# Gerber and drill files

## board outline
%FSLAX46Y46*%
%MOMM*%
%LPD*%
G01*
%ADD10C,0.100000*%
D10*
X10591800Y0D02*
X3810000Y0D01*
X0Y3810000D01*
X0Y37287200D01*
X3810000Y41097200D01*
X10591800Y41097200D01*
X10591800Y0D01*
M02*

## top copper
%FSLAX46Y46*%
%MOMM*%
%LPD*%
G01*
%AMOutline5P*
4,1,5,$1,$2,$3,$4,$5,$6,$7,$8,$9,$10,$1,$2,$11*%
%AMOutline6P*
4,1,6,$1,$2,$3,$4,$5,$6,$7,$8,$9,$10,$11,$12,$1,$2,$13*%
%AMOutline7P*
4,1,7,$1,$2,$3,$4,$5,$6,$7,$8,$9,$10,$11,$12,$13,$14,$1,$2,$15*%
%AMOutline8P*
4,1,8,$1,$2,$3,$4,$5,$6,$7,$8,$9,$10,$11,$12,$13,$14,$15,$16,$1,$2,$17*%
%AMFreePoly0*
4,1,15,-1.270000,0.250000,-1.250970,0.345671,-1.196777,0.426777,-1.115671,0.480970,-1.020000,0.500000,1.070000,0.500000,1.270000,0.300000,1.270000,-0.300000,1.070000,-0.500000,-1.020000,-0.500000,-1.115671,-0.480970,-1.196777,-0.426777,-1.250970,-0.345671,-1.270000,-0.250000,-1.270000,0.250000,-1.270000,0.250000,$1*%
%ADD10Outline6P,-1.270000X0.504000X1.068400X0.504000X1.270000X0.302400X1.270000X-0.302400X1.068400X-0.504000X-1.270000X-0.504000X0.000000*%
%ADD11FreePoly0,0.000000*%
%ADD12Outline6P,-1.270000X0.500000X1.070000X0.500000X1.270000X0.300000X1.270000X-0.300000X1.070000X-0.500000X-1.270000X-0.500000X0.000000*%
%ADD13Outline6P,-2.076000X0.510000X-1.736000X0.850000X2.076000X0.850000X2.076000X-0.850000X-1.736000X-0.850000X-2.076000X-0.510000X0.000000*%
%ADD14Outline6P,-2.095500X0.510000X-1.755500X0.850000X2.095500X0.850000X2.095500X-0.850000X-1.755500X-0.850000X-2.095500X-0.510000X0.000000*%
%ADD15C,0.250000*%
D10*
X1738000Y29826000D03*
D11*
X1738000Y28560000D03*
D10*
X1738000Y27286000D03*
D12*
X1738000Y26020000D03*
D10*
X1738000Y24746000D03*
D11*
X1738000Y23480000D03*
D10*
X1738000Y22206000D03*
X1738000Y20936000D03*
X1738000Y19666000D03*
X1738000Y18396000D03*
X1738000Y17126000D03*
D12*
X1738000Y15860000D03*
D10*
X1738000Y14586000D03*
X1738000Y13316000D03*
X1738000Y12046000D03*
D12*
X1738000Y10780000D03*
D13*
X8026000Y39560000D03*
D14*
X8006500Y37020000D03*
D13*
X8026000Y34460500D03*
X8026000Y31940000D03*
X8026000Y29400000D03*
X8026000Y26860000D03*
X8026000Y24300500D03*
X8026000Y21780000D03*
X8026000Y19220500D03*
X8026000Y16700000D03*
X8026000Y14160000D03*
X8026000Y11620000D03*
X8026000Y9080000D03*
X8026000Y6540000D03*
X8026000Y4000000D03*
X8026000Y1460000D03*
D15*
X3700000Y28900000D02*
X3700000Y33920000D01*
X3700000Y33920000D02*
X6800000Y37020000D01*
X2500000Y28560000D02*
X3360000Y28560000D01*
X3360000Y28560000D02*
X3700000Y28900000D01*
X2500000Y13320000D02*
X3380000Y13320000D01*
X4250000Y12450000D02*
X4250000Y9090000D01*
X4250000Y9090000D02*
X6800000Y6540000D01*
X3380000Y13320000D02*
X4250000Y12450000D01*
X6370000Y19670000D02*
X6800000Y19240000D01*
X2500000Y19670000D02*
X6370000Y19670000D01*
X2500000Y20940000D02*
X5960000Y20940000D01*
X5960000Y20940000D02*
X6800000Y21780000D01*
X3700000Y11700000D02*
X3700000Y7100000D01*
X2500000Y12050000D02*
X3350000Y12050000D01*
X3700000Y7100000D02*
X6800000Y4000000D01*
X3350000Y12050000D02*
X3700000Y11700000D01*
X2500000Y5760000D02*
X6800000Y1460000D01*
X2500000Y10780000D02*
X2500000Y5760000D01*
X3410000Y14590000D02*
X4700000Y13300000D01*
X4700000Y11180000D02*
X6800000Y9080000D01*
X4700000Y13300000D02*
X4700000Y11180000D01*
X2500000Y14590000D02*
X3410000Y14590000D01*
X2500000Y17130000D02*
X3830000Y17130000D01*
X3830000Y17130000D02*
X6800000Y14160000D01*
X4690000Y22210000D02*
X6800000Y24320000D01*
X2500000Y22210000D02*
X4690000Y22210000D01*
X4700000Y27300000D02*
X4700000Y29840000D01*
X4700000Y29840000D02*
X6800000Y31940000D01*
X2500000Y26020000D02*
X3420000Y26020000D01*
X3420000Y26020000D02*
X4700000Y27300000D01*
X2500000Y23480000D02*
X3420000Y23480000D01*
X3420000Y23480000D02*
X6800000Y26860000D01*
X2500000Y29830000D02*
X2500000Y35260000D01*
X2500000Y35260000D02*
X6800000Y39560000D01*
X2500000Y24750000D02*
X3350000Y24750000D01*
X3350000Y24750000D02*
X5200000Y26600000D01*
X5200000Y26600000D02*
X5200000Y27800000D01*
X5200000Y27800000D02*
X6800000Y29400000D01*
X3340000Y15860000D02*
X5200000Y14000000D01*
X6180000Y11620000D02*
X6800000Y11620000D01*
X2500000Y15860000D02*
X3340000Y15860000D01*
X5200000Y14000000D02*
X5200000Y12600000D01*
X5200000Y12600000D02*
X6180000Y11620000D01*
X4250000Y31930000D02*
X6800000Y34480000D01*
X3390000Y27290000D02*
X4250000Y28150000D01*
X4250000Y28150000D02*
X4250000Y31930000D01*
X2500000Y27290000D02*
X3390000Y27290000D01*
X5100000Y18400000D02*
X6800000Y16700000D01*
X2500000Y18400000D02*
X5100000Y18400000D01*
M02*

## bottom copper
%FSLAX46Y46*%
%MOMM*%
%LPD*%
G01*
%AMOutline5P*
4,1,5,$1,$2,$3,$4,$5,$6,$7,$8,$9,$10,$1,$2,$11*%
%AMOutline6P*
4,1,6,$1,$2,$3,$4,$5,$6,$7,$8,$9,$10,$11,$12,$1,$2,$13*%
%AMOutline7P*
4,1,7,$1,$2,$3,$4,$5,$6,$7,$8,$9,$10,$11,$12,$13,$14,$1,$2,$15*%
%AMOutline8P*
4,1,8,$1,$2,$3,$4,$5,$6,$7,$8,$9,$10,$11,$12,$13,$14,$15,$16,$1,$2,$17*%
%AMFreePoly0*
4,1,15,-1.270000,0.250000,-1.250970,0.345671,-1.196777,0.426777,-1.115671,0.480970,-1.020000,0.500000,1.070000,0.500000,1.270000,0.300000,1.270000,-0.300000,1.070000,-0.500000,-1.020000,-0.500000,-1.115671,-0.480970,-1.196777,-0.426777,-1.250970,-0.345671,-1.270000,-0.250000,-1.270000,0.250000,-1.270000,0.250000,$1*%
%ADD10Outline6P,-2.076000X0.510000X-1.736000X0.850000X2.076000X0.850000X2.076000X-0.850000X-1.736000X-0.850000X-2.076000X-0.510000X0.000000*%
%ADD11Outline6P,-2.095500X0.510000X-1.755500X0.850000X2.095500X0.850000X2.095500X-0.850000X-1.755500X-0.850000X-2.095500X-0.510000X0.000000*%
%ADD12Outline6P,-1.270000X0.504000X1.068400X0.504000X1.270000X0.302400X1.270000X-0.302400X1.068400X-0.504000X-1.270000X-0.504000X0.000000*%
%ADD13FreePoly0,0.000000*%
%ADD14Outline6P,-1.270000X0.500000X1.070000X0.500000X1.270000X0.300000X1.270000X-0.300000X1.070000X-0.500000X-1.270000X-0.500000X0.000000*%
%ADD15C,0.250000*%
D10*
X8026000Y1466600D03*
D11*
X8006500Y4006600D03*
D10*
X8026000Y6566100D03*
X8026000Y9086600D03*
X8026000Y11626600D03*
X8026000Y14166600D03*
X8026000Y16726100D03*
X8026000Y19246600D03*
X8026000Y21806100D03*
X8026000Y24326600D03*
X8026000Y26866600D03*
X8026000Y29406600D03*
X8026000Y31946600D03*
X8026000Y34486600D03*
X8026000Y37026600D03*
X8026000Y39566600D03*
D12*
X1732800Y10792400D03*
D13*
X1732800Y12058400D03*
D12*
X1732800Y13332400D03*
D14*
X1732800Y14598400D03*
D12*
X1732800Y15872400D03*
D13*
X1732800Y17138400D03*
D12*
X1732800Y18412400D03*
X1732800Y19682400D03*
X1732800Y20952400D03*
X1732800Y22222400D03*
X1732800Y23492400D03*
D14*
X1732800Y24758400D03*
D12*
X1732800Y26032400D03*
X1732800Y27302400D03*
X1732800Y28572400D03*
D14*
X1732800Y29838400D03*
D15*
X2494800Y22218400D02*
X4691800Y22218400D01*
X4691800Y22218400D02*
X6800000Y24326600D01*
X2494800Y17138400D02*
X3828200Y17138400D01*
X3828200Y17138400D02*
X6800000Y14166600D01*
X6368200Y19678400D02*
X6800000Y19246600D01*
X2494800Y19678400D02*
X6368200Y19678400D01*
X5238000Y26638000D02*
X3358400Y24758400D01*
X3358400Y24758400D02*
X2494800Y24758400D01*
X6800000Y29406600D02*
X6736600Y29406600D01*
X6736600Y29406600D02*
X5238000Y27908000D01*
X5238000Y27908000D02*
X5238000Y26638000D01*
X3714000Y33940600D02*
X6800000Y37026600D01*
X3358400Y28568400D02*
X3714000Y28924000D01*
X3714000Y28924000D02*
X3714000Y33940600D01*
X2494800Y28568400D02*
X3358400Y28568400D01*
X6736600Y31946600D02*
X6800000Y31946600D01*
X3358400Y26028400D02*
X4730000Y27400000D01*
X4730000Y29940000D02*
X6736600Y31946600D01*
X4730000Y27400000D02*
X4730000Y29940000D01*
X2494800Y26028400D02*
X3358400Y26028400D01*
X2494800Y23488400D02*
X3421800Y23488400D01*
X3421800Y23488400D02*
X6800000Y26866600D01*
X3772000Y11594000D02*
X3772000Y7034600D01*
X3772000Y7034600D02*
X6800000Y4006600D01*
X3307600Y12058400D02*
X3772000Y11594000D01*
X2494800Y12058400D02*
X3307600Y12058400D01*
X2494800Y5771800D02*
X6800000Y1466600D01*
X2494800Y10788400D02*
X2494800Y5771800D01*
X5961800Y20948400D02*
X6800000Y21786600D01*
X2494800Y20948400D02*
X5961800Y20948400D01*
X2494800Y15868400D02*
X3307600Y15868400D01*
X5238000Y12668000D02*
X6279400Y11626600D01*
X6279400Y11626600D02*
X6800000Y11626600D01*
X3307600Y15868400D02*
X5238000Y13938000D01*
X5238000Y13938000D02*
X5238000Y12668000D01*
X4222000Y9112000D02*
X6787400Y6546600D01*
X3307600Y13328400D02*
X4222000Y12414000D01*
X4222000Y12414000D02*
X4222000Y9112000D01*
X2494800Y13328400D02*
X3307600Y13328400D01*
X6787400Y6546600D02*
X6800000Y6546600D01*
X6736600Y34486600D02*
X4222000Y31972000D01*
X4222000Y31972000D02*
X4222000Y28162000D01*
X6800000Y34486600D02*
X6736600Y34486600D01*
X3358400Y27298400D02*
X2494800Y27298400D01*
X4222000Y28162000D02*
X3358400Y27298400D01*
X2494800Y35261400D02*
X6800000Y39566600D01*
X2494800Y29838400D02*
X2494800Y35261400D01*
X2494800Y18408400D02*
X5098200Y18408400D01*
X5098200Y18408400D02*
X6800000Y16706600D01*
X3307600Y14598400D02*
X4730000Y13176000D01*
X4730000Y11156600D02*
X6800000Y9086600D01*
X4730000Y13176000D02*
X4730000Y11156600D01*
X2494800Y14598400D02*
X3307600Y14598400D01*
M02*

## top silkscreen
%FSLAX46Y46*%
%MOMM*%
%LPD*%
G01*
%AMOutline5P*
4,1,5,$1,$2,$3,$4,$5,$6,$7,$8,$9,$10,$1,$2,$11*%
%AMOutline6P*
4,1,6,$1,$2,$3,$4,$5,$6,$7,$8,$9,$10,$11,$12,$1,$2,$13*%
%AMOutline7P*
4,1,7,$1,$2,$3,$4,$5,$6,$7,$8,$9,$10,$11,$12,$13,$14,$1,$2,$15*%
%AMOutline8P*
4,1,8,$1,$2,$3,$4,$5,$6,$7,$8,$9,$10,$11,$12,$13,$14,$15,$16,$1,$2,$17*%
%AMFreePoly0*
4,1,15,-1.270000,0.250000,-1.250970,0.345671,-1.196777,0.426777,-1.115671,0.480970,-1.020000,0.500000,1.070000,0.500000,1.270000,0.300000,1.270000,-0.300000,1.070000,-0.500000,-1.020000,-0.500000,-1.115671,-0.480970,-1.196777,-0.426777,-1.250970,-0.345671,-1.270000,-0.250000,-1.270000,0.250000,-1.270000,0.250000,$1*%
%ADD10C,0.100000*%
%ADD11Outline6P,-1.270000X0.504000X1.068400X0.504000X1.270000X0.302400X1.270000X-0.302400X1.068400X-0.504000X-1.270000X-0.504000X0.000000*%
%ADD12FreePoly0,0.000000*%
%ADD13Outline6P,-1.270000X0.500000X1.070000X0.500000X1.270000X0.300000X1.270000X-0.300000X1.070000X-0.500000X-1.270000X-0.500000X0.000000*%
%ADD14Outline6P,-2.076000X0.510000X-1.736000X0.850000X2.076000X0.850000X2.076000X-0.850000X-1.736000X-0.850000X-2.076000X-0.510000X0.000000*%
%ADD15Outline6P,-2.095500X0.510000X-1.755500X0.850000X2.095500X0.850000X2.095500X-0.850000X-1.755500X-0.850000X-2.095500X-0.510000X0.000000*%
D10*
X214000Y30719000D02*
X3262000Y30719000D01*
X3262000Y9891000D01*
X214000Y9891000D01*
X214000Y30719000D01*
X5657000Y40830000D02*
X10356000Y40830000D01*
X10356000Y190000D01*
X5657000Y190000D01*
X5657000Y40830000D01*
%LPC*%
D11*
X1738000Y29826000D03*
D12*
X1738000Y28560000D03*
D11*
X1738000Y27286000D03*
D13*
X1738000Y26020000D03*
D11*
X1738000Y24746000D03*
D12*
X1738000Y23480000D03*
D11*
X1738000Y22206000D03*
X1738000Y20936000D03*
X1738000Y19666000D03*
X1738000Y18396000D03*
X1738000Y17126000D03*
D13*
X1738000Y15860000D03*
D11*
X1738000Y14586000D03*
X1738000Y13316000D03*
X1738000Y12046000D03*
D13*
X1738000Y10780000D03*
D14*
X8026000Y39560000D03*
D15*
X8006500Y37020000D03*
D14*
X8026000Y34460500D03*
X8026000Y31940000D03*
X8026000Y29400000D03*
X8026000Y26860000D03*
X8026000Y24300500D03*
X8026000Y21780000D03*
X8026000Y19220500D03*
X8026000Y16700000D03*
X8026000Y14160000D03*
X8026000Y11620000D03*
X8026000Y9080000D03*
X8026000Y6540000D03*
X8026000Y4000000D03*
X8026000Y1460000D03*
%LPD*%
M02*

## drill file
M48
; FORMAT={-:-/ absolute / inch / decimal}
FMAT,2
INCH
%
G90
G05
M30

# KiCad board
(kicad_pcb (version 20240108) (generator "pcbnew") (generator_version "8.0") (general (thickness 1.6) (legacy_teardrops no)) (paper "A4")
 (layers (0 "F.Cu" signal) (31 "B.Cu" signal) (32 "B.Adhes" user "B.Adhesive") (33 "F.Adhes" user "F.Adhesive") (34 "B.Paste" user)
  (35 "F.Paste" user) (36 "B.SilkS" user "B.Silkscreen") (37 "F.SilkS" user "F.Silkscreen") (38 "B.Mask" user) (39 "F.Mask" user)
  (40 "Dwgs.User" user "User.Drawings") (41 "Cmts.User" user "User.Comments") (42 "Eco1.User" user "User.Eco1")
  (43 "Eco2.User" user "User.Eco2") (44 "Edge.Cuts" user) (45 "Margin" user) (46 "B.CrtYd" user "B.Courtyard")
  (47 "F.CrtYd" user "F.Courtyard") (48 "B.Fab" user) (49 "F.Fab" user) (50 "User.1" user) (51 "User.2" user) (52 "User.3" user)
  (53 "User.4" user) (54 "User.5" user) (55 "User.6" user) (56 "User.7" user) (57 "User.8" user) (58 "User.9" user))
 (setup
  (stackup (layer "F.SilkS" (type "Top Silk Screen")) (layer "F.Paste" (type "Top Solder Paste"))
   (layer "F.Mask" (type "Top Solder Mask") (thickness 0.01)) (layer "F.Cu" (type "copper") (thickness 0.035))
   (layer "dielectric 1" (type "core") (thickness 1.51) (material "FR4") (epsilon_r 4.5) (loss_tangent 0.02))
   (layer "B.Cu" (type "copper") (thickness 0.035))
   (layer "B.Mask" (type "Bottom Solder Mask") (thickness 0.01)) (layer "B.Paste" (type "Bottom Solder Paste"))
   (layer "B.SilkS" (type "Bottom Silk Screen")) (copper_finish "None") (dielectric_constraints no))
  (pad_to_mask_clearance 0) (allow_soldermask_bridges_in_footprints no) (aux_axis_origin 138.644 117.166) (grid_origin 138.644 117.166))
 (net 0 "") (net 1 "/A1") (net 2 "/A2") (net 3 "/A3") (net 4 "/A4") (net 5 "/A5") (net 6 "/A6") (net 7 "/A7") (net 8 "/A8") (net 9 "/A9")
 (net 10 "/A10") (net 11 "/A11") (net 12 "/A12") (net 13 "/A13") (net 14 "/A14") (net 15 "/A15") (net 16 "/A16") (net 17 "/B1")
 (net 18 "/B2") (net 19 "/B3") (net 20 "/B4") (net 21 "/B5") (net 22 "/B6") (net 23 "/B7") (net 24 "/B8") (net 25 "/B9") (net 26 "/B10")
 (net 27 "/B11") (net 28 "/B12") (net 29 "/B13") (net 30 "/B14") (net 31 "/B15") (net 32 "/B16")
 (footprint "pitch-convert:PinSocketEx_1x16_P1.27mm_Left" (layer "F.Cu") (at 139.62 87.336)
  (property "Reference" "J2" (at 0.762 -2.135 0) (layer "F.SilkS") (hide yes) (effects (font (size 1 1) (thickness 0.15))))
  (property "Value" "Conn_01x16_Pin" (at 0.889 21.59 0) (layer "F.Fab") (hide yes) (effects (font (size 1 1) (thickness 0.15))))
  (fp_rect (start -0.762 -0.889) (end 2.286 19.939) (stroke (width 0.1) (type default)) (fill none) (layer "F.SilkS"))
  (pad "1" smd roundrect (at 1.524 0) (size 2.54 1.008) (drill (offset -0.762 0.004)) (layers "F.Cu" "F.Paste" "F.Mask")
   (roundrect_rratio 0) (chamfer_ratio 0.2) (chamfer top_right bottom_right) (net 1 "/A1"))
  (pad "2" smd roundrect (at 1.524 1.27) (size 2.54 1) (drill (offset -0.762 0)) (layers "F.Cu" "F.Paste" "F.Mask") (roundrect_rratio 0.25)
   (chamfer_ratio 0.2) (chamfer top_right bottom_right) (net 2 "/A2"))
  (pad "3" smd roundrect (at 1.524 2.54) (size 2.54 1.008) (drill (offset -0.762 0.004)) (layers "F.Cu" "F.Paste" "F.Mask")
   (roundrect_rratio 0) (chamfer_ratio 0.2) (chamfer top_right bottom_right) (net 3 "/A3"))
  (pad "4" smd roundrect (at 1.524 3.81) (size 2.54 1) (drill (offset -0.762 0)) (layers "F.Cu" "F.Paste" "F.Mask") (roundrect_rratio 0)
   (chamfer_ratio 0.2) (chamfer top_right bottom_right) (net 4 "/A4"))
  (pad "5" smd roundrect (at 1.524 5.08) (size 2.54 1.008) (drill (offset -0.762 0.004)) (layers "F.Cu" "F.Paste" "F.Mask")
   (roundrect_rratio 0) (chamfer_ratio 0.2) (chamfer top_right bottom_right) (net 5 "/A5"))
  (pad "6" smd roundrect (at 1.524 6.35) (size 2.54 1) (drill (offset -0.762 0)) (layers "F.Cu" "F.Paste" "F.Mask") (roundrect_rratio 0.25)
   (chamfer_ratio 0.2) (chamfer top_right bottom_right) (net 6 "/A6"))
  (pad "7" smd roundrect (at 1.524 7.62) (size 2.54 1.008) (drill (offset -0.762 0.004)) (layers "F.Cu" "F.Paste" "F.Mask")
   (roundrect_rratio 0) (chamfer_ratio 0.2) (chamfer top_right bottom_right) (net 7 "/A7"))
  (pad "8" smd roundrect (at 1.524 8.89) (size 2.54 1.008) (drill (offset -0.762 0.004)) (layers "F.Cu" "F.Paste" "F.Mask")
   (roundrect_rratio 0) (chamfer_ratio 0.2) (chamfer top_right bottom_right) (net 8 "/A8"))
  (pad "9" smd roundrect (at 1.524 10.16) (size 2.54 1.008) (drill (offset -0.762 0.004)) (layers "F.Cu" "F.Paste" "F.Mask")
   (roundrect_rratio 0) (chamfer_ratio 0.2) (chamfer top_right bottom_right) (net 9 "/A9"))
  (pad "10" smd roundrect (at 1.524 11.43) (size 2.54 1.008) (drill (offset -0.762 0.004)) (layers "F.Cu" "F.Paste" "F.Mask")
   (roundrect_rratio 0) (chamfer_ratio 0.2) (chamfer top_right bottom_right) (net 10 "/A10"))
  (pad "11" smd roundrect (at 1.524 12.7) (size 2.54 1.008) (drill (offset -0.762 0.004)) (layers "F.Cu" "F.Paste" "F.Mask")
   (roundrect_rratio 0) (chamfer_ratio 0.2) (chamfer top_right bottom_right) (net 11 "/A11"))
  (pad "12" smd roundrect (at 1.524 13.97) (size 2.54 1) (drill (offset -0.762 0)) (layers "F.Cu" "F.Paste" "F.Mask") (roundrect_rratio 0)
   (chamfer_ratio 0.2) (chamfer top_right bottom_right) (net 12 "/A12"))
  (pad "13" smd roundrect (at 1.524 15.24) (size 2.54 1.008) (drill (offset -0.762 0.004)) (layers "F.Cu" "F.Paste" "F.Mask")
   (roundrect_rratio 0) (chamfer_ratio 0.2) (chamfer top_right bottom_right) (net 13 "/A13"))
  (pad "14" smd roundrect (at 1.524 16.51) (size 2.54 1.008) (drill (offset -0.762 0.004)) (layers "F.Cu" "F.Paste" "F.Mask")
   (roundrect_rratio 0) (chamfer_ratio 0.2) (chamfer top_right bottom_right) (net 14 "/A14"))
  (pad "15" smd roundrect (at 1.524 17.78) (size 2.54 1.008) (drill (offset -0.762 0.004)) (layers "F.Cu" "F.Paste" "F.Mask")
   (roundrect_rratio 0) (chamfer_ratio 0.2) (chamfer top_right bottom_right) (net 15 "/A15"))
  (pad "16" smd roundrect (at 1.524 19.05) (size 2.54 1) (drill (offset -0.762 0)) (layers "F.Cu" "F.Paste" "F.Mask") (roundrect_rratio 0)
   (chamfer_ratio 0.2) (chamfer top_right bottom_right) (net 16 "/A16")))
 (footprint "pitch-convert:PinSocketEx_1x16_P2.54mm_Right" (layer "F.Cu") (at 145.444 77.606)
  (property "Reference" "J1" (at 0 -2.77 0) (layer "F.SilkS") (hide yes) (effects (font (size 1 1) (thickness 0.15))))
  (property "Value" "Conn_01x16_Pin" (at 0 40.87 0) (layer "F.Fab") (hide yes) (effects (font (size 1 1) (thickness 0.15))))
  (fp_rect (start -1.143 -1.27) (end 3.556 39.37) (stroke (width 0.1) (type default)) (fill none) (layer "F.SilkS"))
  (pad "1" smd roundrect (at 0 0) (size 4.152 1.7) (drill (offset 1.226 0)) (layers "F.Cu" "F.Paste" "F.Mask") (roundrect_rratio 0)
   (chamfer_ratio 0.2) (chamfer top_left bottom_left) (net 1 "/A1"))
  (pad "2" smd roundrect (at 0 2.54) (size 4.191 1.7) (drill (offset 1.2065 0)) (layers "F.Cu" "F.Paste" "F.Mask") (roundrect_rratio 0)
   (chamfer_ratio 0.2) (chamfer top_left bottom_left) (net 2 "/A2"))
  (pad "3" smd roundrect (at 0 5.08) (size 4.152 1.7) (drill (offset 1.226 0.0195)) (layers "F.Cu" "F.Paste" "F.Mask") (roundrect_rratio 0)
   (chamfer_ratio 0.2) (chamfer top_left bottom_left) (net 3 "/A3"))
  (pad "4" smd roundrect (at 0 7.62) (size 4.152 1.7) (drill (offset 1.226 0)) (layers "F.Cu" "F.Paste" "F.Mask") (roundrect_rratio 0)
   (chamfer_ratio 0.2) (chamfer top_left bottom_left) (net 4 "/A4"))
  (pad "5" smd roundrect (at 0 10.16) (size 4.152 1.7) (drill (offset 1.226 0)) (layers "F.Cu" "F.Paste" "F.Mask") (roundrect_rratio 0)
   (chamfer_ratio 0.2) (chamfer top_left bottom_left) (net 5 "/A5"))
  (pad "6" smd roundrect (at 0 12.7) (size 4.152 1.7) (drill (offset 1.226 0)) (layers "F.Cu" "F.Paste" "F.Mask") (roundrect_rratio 0)
   (chamfer_ratio 0.2) (chamfer top_left bottom_left) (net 6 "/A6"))
  (pad "7" smd roundrect (at 0 15.24) (size 4.152 1.7) (drill (offset 1.226 0.0195)) (layers "F.Cu" "F.Paste" "F.Mask") (roundrect_rratio 0)
   (chamfer_ratio 0.2) (chamfer top_left bottom_left) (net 7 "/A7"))
  (pad "8" smd roundrect (at 0 17.78) (size 4.152 1.7) (drill (offset 1.226 0)) (layers "F.Cu" "F.Paste" "F.Mask") (roundrect_rratio 0)
   (chamfer_ratio 0.2) (chamfer top_left bottom_left) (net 8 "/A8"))
  (pad "9" smd roundrect (at 0 20.32) (size 4.152 1.7) (drill (offset 1.226 0.0195)) (layers "F.Cu" "F.Paste" "F.Mask") (roundrect_rratio 0)
   (chamfer_ratio 0.2) (chamfer top_left bottom_left) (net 9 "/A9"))
  (pad "10" smd roundrect (at 0 22.86) (size 4.152 1.7) (drill (offset 1.226 0)) (layers "F.Cu" "F.Paste" "F.Mask") (roundrect_rratio 0)
   (chamfer_ratio 0.2) (chamfer top_left bottom_left) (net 10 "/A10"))
  (pad "11" smd roundrect (at 0 25.4) (size 4.152 1.7) (drill (offset 1.226 0)) (layers "F.Cu" "F.Paste" "F.Mask") (roundrect_rratio 0)
   (chamfer_ratio 0.2) (chamfer top_left bottom_left) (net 11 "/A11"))
  (pad "12" smd roundrect (at 0 27.94) (size 4.152 1.7) (drill (offset 1.226 0)) (layers "F.Cu" "F.Paste" "F.Mask") (roundrect_rratio 0)
   (chamfer_ratio 0.2) (chamfer top_left bottom_left) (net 12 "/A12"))
  (pad "13" smd roundrect (at 0 30.48) (size 4.152 1.7) (drill (offset 1.226 0)) (layers "F.Cu" "F.Paste" "F.Mask") (roundrect_rratio 0)
   (chamfer_ratio 0.2) (chamfer top_left bottom_left) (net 13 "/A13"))
  (pad "14" smd roundrect (at 0 33.02) (size 4.152 1.7) (drill (offset 1.226 0)) (layers "F.Cu" "F.Paste" "F.Mask") (roundrect_rratio 0)
   (chamfer_ratio 0.2) (chamfer top_left bottom_left) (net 14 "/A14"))
  (pad "15" smd roundrect (at 0 35.56) (size 4.152 1.7) (drill (offset 1.226 0)) (layers "F.Cu" "F.Paste" "F.Mask") (roundrect_rratio 0)
   (chamfer_ratio 0.2) (chamfer top_left bottom_left) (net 15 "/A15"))
  (pad "16" smd roundrect (at 0 38.1) (size 4.152 1.7) (drill (offset 1.226 0)) (layers "F.Cu" "F.Paste" "F.Mask") (roundrect_rratio 0)
   (chamfer_ratio 0.2) (chamfer top_left bottom_left) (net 16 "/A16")))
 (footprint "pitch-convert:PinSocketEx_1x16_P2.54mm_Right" (layer "B.Cu") (at 145.444 115.6994)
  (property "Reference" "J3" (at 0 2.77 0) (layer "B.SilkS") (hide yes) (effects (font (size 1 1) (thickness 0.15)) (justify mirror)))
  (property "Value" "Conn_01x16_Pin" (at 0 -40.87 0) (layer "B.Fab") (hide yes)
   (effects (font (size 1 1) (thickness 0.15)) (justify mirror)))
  (pad "1" smd roundrect (at 0 0) (size 4.152 1.7) (drill (offset 1.226 0)) (layers "B.Cu" "B.Paste" "B.Mask") (roundrect_rratio 0)
   (chamfer_ratio 0.2) (chamfer top_left bottom_left) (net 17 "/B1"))
  (pad "2" smd roundrect (at 0 -2.54) (size 4.191 1.7) (drill (offset 1.2065 0)) (layers "B.Cu" "B.Paste" "B.Mask") (roundrect_rratio 0)
   (chamfer_ratio 0.2) (chamfer top_left bottom_left) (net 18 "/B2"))
  (pad "3" smd roundrect (at 0 -5.08) (size 4.152 1.7) (drill (offset 1.226 -0.0195)) (layers "B.Cu" "B.Paste" "B.Mask")
   (roundrect_rratio 0) (chamfer_ratio 0.2) (chamfer top_left bottom_left) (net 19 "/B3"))
  (pad "4" smd roundrect (at 0 -7.62) (size 4.152 1.7) (drill (offset 1.226 0)) (layers "B.Cu" "B.Paste" "B.Mask") (roundrect_rratio 0)
   (chamfer_ratio 0.2) (chamfer top_left bottom_left) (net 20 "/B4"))
  (pad "5" smd roundrect (at 0 -10.16) (size 4.152 1.7) (drill (offset 1.226 0)) (layers "B.Cu" "B.Paste" "B.Mask") (roundrect_rratio 0)
   (chamfer_ratio 0.2) (chamfer top_left bottom_left) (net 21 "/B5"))
  (pad "6" smd roundrect (at 0 -12.7) (size 4.152 1.7) (drill (offset 1.226 0)) (layers "B.Cu" "B.Paste" "B.Mask") (roundrect_rratio 0)
   (chamfer_ratio 0.2) (chamfer top_left bottom_left) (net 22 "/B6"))
  (pad "7" smd roundrect (at 0 -15.24) (size 4.152 1.7) (drill (offset 1.226 -0.0195)) (layers "B.Cu" "B.Paste" "B.Mask")
   (roundrect_rratio 0) (chamfer_ratio 0.2) (chamfer top_left bottom_left) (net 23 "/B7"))
  (pad "8" smd roundrect (at 0 -17.78) (size 4.152 1.7) (drill (offset 1.226 0)) (layers "B.Cu" "B.Paste" "B.Mask") (roundrect_rratio 0)
   (chamfer_ratio 0.2) (chamfer top_left bottom_left) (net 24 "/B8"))
  (pad "9" smd roundrect (at 0 -20.32) (size 4.152 1.7) (drill (offset 1.226 -0.0195)) (layers "B.Cu" "B.Paste" "B.Mask")
   (roundrect_rratio 0) (chamfer_ratio 0.2) (chamfer top_left bottom_left) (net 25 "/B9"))
  (pad "10" smd roundrect (at 0 -22.86) (size 4.152 1.7) (drill (offset 1.226 0)) (layers "B.Cu" "B.Paste" "B.Mask") (roundrect_rratio 0)
   (chamfer_ratio 0.2) (chamfer top_left bottom_left) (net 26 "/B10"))
  (pad "11" smd roundrect (at 0 -25.4) (size 4.152 1.7) (drill (offset 1.226 0)) (layers "B.Cu" "B.Paste" "B.Mask") (roundrect_rratio 0)
   (chamfer_ratio 0.2) (chamfer top_left bottom_left) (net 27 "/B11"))
  (pad "12" smd roundrect (at 0 -27.94) (size 4.152 1.7) (drill (offset 1.226 0)) (layers "B.Cu" "B.Paste" "B.Mask") (roundrect_rratio 0)
   (chamfer_ratio 0.2) (chamfer top_left bottom_left) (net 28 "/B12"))
  (pad "13" smd roundrect (at 0 -30.48) (size 4.152 1.7) (drill (offset 1.226 0)) (layers "B.Cu" "B.Paste" "B.Mask") (roundrect_rratio 0)
   (chamfer_ratio 0.2) (chamfer top_left bottom_left) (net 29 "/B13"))
  (pad "14" smd roundrect (at 0 -33.02) (size 4.152 1.7) (drill (offset 1.226 0)) (layers "B.Cu" "B.Paste" "B.Mask") (roundrect_rratio 0)
   (chamfer_ratio 0.2) (chamfer top_left bottom_left) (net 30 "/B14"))
  (pad "15" smd roundrect (at 0 -35.56) (size 4.152 1.7) (drill (offset 1.226 0)) (layers "B.Cu" "B.Paste" "B.Mask") (roundrect_rratio 0)
   (chamfer_ratio 0.2) (chamfer top_left bottom_left) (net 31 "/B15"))
  (pad "16" smd roundrect (at 0 -38.1) (size 4.152 1.7) (drill (offset 1.226 0)) (layers "B.Cu" "B.Paste" "B.Mask") (roundrect_rratio 0)
   (chamfer_ratio 0.2) (chamfer top_left bottom_left) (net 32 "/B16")))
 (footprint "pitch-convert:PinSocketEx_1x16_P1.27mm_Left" (layer "B.Cu") (at 139.6148 106.3776)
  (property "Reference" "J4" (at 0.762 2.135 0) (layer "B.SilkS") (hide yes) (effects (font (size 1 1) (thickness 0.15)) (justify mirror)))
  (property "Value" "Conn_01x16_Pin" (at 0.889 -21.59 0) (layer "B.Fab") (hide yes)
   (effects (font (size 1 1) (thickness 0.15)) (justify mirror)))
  (pad "1" smd roundrect (at 1.524 0) (size 2.54 1.008) (drill (offset -0.762 -0.004)) (layers "B.Cu" "B.Paste" "B.Mask")
   (roundrect_rratio 0) (chamfer_ratio 0.2) (chamfer top_right bottom_right) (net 17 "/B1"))
  (pad "2" smd roundrect (at 1.524 -1.27) (size 2.54 1) (drill (offset -0.762 0)) (layers "B.Cu" "B.Paste" "B.Mask") (roundrect_rratio 0.25)
   (chamfer_ratio 0.2) (chamfer top_right bottom_right) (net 18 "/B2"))
  (pad "3" smd roundrect (at 1.524 -2.54) (size 2.54 1.008) (drill (offset -0.762 -0.004)) (layers "B.Cu" "B.Paste" "B.Mask")
   (roundrect_rratio 0) (chamfer_ratio 0.2) (chamfer top_right bottom_right) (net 19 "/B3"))
  (pad "4" smd roundrect (at 1.524 -3.81) (size 2.54 1) (drill (offset -0.762 0)) (layers "B.Cu" "B.Paste" "B.Mask") (roundrect_rratio 0)
   (chamfer_ratio 0.2) (chamfer top_right bottom_right) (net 20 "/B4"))
  (pad "5" smd roundrect (at 1.524 -5.08) (size 2.54 1.008) (drill (offset -0.762 -0.004)) (layers "B.Cu" "B.Paste" "B.Mask")
   (roundrect_rratio 0) (chamfer_ratio 0.2) (chamfer top_right bottom_right) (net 21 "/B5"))
  (pad "6" smd roundrect (at 1.524 -6.35) (size 2.54 1) (drill (offset -0.762 0)) (layers "B.Cu" "B.Paste" "B.Mask") (roundrect_rratio 0.25)
   (chamfer_ratio 0.2) (chamfer top_right bottom_right) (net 22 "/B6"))
  (pad "7" smd roundrect (at 1.524 -7.62) (size 2.54 1.008) (drill (offset -0.762 -0.004)) (layers "B.Cu" "B.Paste" "B.Mask")
   (roundrect_rratio 0) (chamfer_ratio 0.2) (chamfer top_right bottom_right) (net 23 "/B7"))
  (pad "8" smd roundrect (at 1.524 -8.89) (size 2.54 1.008) (drill (offset -0.762 -0.004)) (layers "B.Cu" "B.Paste" "B.Mask")
   (roundrect_rratio 0) (chamfer_ratio 0.2) (chamfer top_right bottom_right) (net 24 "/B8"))
  (pad "9" smd roundrect (at 1.524 -10.16) (size 2.54 1.008) (drill (offset -0.762 -0.004)) (layers "B.Cu" "B.Paste" "B.Mask")
   (roundrect_rratio 0) (chamfer_ratio 0.2) (chamfer top_right bottom_right) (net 25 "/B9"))
  (pad "10" smd roundrect (at 1.524 -11.43) (size 2.54 1.008) (drill (offset -0.762 -0.004)) (layers "B.Cu" "B.Paste" "B.Mask")
   (roundrect_rratio 0) (chamfer_ratio 0.2) (chamfer top_right bottom_right) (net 26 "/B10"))
  (pad "11" smd roundrect (at 1.524 -12.7) (size 2.54 1.008) (drill (offset -0.762 -0.004)) (layers "B.Cu" "B.Paste" "B.Mask")
   (roundrect_rratio 0) (chamfer_ratio 0.2) (chamfer top_right bottom_right) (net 27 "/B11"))
  (pad "12" smd roundrect (at 1.524 -13.97) (size 2.54 1) (drill (offset -0.762 0)) (layers "B.Cu" "B.Paste" "B.Mask") (roundrect_rratio 0)
   (chamfer_ratio 0.2) (chamfer top_right bottom_right) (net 28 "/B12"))
  (pad "13" smd roundrect (at 1.524 -15.24) (size 2.54 1.008) (drill (offset -0.762 -0.004)) (layers "B.Cu" "B.Paste" "B.Mask")
   (roundrect_rratio 0) (chamfer_ratio 0.2) (chamfer top_right bottom_right) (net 29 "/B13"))
  (pad "14" smd roundrect (at 1.524 -16.51) (size 2.54 1.008) (drill (offset -0.762 -0.004)) (layers "B.Cu" "B.Paste" "B.Mask")
   (roundrect_rratio 0) (chamfer_ratio 0.2) (chamfer top_right bottom_right) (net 30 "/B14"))
  (pad "15" smd roundrect (at 1.524 -17.78) (size 2.54 1.008) (drill (offset -0.762 -0.004)) (layers "B.Cu" "B.Paste" "B.Mask")
   (roundrect_rratio 0) (chamfer_ratio 0.2) (chamfer top_right bottom_right) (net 31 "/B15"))
  (pad "16" smd roundrect (at 1.524 -19.05) (size 2.54 1) (drill (offset -0.762 0)) (layers "B.Cu" "B.Paste" "B.Mask") (roundrect_rratio 0)
   (chamfer_ratio 0.2) (chamfer top_right bottom_right) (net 32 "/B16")))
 (gr_poly
  (pts (xy 149.2358 76.0688) (xy 142.454 76.0688) (xy 138.644 79.8788) (xy 138.644 113.356) (xy 142.454 117.166) (xy 149.2358 117.166))
  (stroke (width 0.1) (type solid)) (fill none) (layer "Edge.Cuts"))
 (segment (start 142.344 88.266) (end 142.344 83.246) (width 0.25) (layer "F.Cu") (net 2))
 (segment (start 142.344 83.246) (end 145.444 80.146) (width 0.25) (layer "F.Cu") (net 2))
 (segment (start 141.144 88.606) (end 142.004 88.606) (width 0.25) (layer "F.Cu") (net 2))
 (segment (start 142.004 88.606) (end 142.344 88.266) (width 0.25) (layer "F.Cu") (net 2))
 (segment (start 141.144 103.846) (end 142.024 103.846) (width 0.25) (layer "F.Cu") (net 14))
 (segment (start 142.894 104.716) (end 142.894 108.076) (width 0.25) (layer "F.Cu") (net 14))
 (segment (start 142.894 108.076) (end 145.444 110.626) (width 0.25) (layer "F.Cu") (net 14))
 (segment (start 142.024 103.846) (end 142.894 104.716) (width 0.25) (layer "F.Cu") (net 14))
 (segment (start 145.014 97.496) (end 145.444 97.926) (width 0.25) (layer "F.Cu") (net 9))
 (segment (start 141.144 97.496) (end 145.014 97.496) (width 0.25) (layer "F.Cu") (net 9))
 (segment (start 141.144 96.226) (end 144.604 96.226) (width 0.25) (layer "F.Cu") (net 8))
 (segment (start 144.604 96.226) (end 145.444 95.386) (width 0.25) (layer "F.Cu") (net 8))
 (segment (start 142.344 105.466) (end 142.344 110.066) (width 0.25) (layer "F.Cu") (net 15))
 (segment (start 141.144 105.116) (end 141.994 105.116) (width 0.25) (layer "F.Cu") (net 15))
 (segment (start 142.344 110.066) (end 145.444 113.166) (width 0.25) (layer "F.Cu") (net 15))
 (segment (start 141.994 105.116) (end 142.344 105.466) (width 0.25) (layer "F.Cu") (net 15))
 (segment (start 141.144 111.406) (end 145.444 115.706) (width 0.25) (layer "F.Cu") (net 16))
 (segment (start 141.144 106.386) (end 141.144 111.406) (width 0.25) (layer "F.Cu") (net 16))
 (segment (start 142.054 102.576) (end 143.344 103.866) (width 0.25) (layer "F.Cu") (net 13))
 (segment (start 143.344 105.986) (end 145.444 108.086) (width 0.25) (layer "F.Cu") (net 13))
 (segment (start 143.344 103.866) (end 143.344 105.986) (width 0.25) (layer "F.Cu") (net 13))
 (segment (start 141.144 102.576) (end 142.054 102.576) (width 0.25) (layer "F.Cu") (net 13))
 (segment (start 141.144 100.036) (end 142.474 100.036) (width 0.25) (layer "F.Cu") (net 11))
 (segment (start 142.474 100.036) (end 145.444 103.006) (width 0.25) (layer "F.Cu") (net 11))
 (segment (start 143.334 94.956) (end 145.444 92.846) (width 0.25) (layer "F.Cu") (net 7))
 (segment (start 141.144 94.956) (end 143.334 94.956) (width 0.25) (layer "F.Cu") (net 7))
 (segment (start 143.344 89.866) (end 143.344 87.326) (width 0.25) (layer "F.Cu") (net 4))
 (segment (start 143.344 87.326) (end 145.444 85.226) (width 0.25) (layer "F.Cu") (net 4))
 (segment (start 141.144 91.146) (end 142.064 91.146) (width 0.25) (layer "F.Cu") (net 4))
 (segment (start 142.064 91.146) (end 143.344 89.866) (width 0.25) (layer "F.Cu") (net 4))
 (segment (start 141.144 93.686) (end 142.064 93.686) (width 0.25) (layer "F.Cu") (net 6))
 (segment (start 142.064 93.686) (end 145.444 90.306) (width 0.25) (layer "F.Cu") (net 6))
 (segment (start 141.144 87.336) (end 141.144 81.906) (width 0.25) (layer "F.Cu") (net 1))
 (segment (start 141.144 81.906) (end 145.444 77.606) (width 0.25) (layer "F.Cu") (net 1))
 (segment (start 141.144 92.416) (end 141.994 92.416) (width 0.25) (layer "F.Cu") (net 5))
 (segment (start 141.994 92.416) (end 143.844 90.566) (width 0.25) (layer "F.Cu") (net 5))
 (segment (start 143.844 90.566) (end 143.844 89.366) (width 0.25) (layer "F.Cu") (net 5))
 (segment (start 143.844 89.366) (end 145.444 87.766) (width 0.25) (layer "F.Cu") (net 5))
 (segment (start 141.984 101.306) (end 143.844 103.166) (width 0.25) (layer "F.Cu") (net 12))
 (segment (start 144.824 105.546) (end 145.444 105.546) (width 0.25) (layer "F.Cu") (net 12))
 (segment (start 141.144 101.306) (end 141.984 101.306) (width 0.25) (layer "F.Cu") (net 12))
 (segment (start 143.844 103.166) (end 143.844 104.566) (width 0.25) (layer "F.Cu") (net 12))
 (segment (start 143.844 104.566) (end 144.824 105.546) (width 0.25) (layer "F.Cu") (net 12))
 (segment (start 142.894 85.236) (end 145.444 82.686) (width 0.25) (layer "F.Cu") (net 3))
 (segment (start 142.034 89.876) (end 142.894 89.016) (width 0.25) (layer "F.Cu") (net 3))
 (segment (start 142.894 89.016) (end 142.894 85.236) (width 0.25) (layer "F.Cu") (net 3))
 (segment (start 141.144 89.876) (end 142.034 89.876) (width 0.25) (layer "F.Cu") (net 3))
 (segment (start 143.744 98.766) (end 145.444 100.466) (width 0.25) (layer "F.Cu") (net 10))
 (segment (start 141.144 98.766) (end 143.744 98.766) (width 0.25) (layer "F.Cu") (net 10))
 (segment (start 141.1388 94.9476) (end 143.3358 94.9476) (width 0.25) (layer "B.Cu") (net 26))
 (segment (start 143.3358 94.9476) (end 145.444 92.8394) (width 0.25) (layer "B.Cu") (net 26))
 (segment (start 141.1388 100.0276) (end 142.4722 100.0276) (width 0.25) (layer "B.Cu") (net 22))
 (segment (start 142.4722 100.0276) (end 145.444 102.9994) (width 0.25) (layer "B.Cu") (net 22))
 (segment (start 145.0122 97.4876) (end 145.444 97.9194) (width 0.25) (layer "B.Cu") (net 24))
 (segment (start 141.1388 97.4876) (end 145.0122 97.4876) (width 0.25) (layer "B.Cu") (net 24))
 (segment (start 143.882 90.528) (end 142.0024 92.4076) (width 0.25) (layer "B.Cu") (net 28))
 (segment (start 142.0024 92.4076) (end 141.1388 92.4076) (width 0.25) (layer "B.Cu") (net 28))
 (segment (start 145.444 87.7594) (end 145.3806 87.7594) (width 0.25) (layer "B.Cu") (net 28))
 (segment (start 145.3806 87.7594) (end 143.882 89.258) (width 0.25) (layer "B.Cu") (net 28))
 (segment (start 143.882 89.258) (end 143.882 90.528) (width 0.25) (layer "B.Cu") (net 28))
 (segment (start 142.358 83.2254) (end 145.444 80.1394) (width 0.25) (layer "B.Cu") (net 31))
 (segment (start 142.0024 88.5976) (end 142.358 88.242) (width 0.25) (layer "B.Cu") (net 31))
 (segment (start 142.358 88.242) (end 142.358 83.2254) (width 0.25) (layer "B.Cu") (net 31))
 (segment (start 141.1388 88.5976) (end 142.0024 88.5976) (width 0.25) (layer "B.Cu") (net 31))
 (segment (start 145.3806 85.2194) (end 145.444 85.2194) (width 0.25) (layer "B.Cu") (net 29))
 (segment (start 142.0024 91.1376) (end 143.374 89.766) (width 0.25) (layer "B.Cu") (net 29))
 (segment (start 143.374 87.226) (end 145.3806 85.2194) (width 0.25) (layer "B.Cu") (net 29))
 (segment (start 143.374 89.766) (end 143.374 87.226) (width 0.25) (layer "B.Cu") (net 29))
 (segment (start 141.1388 91.1376) (end 142.0024 91.1376) (width 0.25) (layer "B.Cu") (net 29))
 (segment (start 141.1388 93.6776) (end 142.0658 93.6776) (width 0.25) (layer "B.Cu") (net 27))
 (segment (start 142.0658 93.6776) (end 145.444 90.2994) (width 0.25) (layer "B.Cu") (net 27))
 (segment (start 142.416 105.572) (end 142.416 110.1314) (width 0.25) (layer "B.Cu") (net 18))
 (segment (start 142.416 110.1314) (end 145.444 113.1594) (width 0.25) (layer "B.Cu") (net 18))
 (segment (start 141.9516 105.1076) (end 142.416 105.572) (width 0.25) (layer "B.Cu") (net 18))
 (segment (start 141.1388 105.1076) (end 141.9516 105.1076) (width 0.25) (layer "B.Cu") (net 18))
 (segment (start 141.1388 111.3942) (end 145.444 115.6994) (width 0.25) (layer "B.Cu") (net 17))
 (segment (start 141.1388 106.3776) (end 141.1388 111.3942) (width 0.25) (layer "B.Cu") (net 17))
 (segment (start 144.6058 96.2176) (end 145.444 95.3794) (width 0.25) (layer "B.Cu") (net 25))
 (segment (start 141.1388 96.2176) (end 144.6058 96.2176) (width 0.25) (layer "B.Cu") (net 25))
 (segment (start 141.1388 101.2976) (end 141.9516 101.2976) (width 0.25) (layer "B.Cu") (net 21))
 (segment (start 143.882 104.498) (end 144.9234 105.5394) (width 0.25) (layer "B.Cu") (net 21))
 (segment (start 144.9234 105.5394) (end 145.444 105.5394) (width 0.25) (layer "B.Cu") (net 21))
 (segment (start 141.9516 101.2976) (end 143.882 103.228) (width 0.25) (layer "B.Cu") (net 21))
 (segment (start 143.882 103.228) (end 143.882 104.498) (width 0.25) (layer "B.Cu") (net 21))
 (segment (start 142.866 108.054) (end 145.4314 110.6194) (width 0.25) (layer "B.Cu") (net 19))
 (segment (start 141.9516 103.8376) (end 142.866 104.752) (width 0.25) (layer "B.Cu") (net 19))
 (segment (start 142.866 104.752) (end 142.866 108.054) (width 0.25) (layer "B.Cu") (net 19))
 (segment (start 141.1388 103.8376) (end 141.9516 103.8376) (width 0.25) (layer "B.Cu") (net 19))
 (segment (start 145.4314 110.6194) (end 145.444 110.6194) (width 0.25) (layer "B.Cu") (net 19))
 (segment (start 145.3806 82.6794) (end 142.866 85.194) (width 0.25) (layer "B.Cu") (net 30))
 (segment (start 142.866 85.194) (end 142.866 89.004) (width 0.25) (layer "B.Cu") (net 30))
 (segment (start 145.444 82.6794) (end 145.3806 82.6794) (width 0.25) (layer "B.Cu") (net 30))
 (segment (start 142.0024 89.8676) (end 141.1388 89.8676) (width 0.25) (layer "B.Cu") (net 30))
 (segment (start 142.866 89.004) (end 142.0024 89.8676) (width 0.25) (layer "B.Cu") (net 30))
 (segment (start 141.1388 81.9046) (end 145.444 77.5994) (width 0.25) (layer "B.Cu") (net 32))
 (segment (start 141.1388 87.3276) (end 141.1388 81.9046) (width 0.25) (layer "B.Cu") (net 32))
 (segment (start 141.1388 98.7576) (end 143.7422 98.7576) (width 0.25) (layer "B.Cu") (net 23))
 (segment (start 143.7422 98.7576) (end 145.444 100.4594) (width 0.25) (layer "B.Cu") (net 23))
 (segment (start 141.9516 102.5676) (end 143.374 103.99) (width 0.25) (layer "B.Cu") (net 20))
 (segment (start 143.374 106.0094) (end 145.444 108.0794) (width 0.25) (layer "B.Cu") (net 20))
 (segment (start 143.374 103.99) (end 143.374 106.0094) (width 0.25) (layer "B.Cu") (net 20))
 (segment (start 141.1388 102.5676) (end 141.9516 102.5676) (width 0.25) (layer "B.Cu") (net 20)))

